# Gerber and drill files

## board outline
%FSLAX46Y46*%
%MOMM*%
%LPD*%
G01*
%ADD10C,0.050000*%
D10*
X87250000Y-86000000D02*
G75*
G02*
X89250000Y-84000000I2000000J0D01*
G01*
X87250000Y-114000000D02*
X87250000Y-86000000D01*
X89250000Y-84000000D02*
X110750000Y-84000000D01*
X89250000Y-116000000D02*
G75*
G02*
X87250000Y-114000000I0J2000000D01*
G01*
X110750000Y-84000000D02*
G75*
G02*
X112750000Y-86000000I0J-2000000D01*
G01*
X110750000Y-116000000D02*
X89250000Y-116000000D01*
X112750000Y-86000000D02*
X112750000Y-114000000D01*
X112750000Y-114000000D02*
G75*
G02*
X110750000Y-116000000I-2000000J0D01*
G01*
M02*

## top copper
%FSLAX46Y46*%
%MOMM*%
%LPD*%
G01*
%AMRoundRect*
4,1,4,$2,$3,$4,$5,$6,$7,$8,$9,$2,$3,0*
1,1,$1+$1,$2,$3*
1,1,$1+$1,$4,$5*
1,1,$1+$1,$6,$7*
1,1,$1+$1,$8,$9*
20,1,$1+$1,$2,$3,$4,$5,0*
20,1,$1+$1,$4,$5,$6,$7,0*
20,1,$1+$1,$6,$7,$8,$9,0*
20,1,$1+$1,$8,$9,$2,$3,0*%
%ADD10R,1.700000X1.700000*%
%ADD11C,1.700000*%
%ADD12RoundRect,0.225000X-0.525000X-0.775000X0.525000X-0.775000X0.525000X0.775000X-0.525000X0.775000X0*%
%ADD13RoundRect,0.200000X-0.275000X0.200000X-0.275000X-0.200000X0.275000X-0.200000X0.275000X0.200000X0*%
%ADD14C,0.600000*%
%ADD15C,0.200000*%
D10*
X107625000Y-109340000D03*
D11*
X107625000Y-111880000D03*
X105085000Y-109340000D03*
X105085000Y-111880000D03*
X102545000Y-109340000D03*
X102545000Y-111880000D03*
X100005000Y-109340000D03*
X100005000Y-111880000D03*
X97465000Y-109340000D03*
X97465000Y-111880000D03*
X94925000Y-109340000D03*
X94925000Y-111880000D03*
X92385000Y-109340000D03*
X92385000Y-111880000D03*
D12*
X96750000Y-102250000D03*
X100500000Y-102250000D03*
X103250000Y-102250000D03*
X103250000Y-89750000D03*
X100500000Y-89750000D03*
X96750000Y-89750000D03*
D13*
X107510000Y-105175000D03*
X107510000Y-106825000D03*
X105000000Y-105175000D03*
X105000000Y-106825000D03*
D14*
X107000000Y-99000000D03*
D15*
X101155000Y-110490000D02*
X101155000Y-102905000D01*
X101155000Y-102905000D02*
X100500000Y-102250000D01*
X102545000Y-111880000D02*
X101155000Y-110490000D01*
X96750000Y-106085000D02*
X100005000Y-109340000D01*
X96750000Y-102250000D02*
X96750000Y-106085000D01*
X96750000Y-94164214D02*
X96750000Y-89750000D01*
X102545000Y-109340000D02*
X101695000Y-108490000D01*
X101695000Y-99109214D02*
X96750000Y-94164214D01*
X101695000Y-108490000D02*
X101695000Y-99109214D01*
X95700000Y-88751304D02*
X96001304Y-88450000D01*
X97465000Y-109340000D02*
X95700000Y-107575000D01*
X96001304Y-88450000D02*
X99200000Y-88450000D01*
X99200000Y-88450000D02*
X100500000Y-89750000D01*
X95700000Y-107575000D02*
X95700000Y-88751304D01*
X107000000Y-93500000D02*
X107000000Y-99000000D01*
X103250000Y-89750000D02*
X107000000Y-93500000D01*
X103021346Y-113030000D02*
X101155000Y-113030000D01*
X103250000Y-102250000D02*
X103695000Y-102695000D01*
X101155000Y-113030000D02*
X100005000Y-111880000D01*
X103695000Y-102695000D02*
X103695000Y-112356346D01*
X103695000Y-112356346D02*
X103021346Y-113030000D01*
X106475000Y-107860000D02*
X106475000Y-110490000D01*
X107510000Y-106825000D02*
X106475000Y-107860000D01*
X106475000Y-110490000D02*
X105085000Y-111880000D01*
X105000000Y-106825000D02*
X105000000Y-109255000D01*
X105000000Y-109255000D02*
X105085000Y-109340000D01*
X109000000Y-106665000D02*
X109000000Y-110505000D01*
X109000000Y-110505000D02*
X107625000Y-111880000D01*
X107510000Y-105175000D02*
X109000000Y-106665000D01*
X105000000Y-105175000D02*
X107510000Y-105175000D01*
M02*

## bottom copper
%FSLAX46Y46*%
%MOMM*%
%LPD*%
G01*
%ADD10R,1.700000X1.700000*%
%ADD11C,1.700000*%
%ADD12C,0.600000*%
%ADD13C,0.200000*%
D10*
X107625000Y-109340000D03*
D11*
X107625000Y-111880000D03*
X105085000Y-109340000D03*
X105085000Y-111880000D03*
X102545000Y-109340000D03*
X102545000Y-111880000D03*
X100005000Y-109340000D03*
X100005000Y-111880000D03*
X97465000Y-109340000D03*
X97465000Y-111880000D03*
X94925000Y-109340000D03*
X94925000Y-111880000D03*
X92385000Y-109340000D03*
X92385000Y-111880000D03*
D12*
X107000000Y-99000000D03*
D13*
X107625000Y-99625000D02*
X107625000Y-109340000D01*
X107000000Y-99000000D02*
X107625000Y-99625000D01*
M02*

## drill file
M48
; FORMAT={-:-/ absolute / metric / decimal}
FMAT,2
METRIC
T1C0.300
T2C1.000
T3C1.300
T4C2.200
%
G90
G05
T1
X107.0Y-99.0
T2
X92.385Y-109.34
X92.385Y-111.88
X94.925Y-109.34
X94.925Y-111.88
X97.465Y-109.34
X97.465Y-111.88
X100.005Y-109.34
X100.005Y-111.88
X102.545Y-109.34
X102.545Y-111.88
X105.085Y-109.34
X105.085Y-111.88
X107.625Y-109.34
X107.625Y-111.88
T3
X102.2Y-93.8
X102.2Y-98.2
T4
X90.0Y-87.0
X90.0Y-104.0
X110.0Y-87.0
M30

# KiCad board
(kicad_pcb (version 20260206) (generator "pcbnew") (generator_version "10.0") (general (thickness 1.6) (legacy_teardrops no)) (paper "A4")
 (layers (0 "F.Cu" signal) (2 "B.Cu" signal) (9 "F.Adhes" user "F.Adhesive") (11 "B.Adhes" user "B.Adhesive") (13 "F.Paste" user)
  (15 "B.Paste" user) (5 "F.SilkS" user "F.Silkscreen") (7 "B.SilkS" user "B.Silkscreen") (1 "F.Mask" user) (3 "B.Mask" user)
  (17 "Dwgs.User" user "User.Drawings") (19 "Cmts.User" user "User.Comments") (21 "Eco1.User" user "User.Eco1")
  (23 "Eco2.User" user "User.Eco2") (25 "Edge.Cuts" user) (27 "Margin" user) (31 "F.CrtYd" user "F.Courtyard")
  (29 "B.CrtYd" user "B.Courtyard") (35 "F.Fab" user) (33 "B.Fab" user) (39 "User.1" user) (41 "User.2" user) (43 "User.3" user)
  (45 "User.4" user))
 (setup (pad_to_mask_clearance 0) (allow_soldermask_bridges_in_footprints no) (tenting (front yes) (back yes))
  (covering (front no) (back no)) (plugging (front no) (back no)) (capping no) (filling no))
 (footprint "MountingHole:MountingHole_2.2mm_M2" (layer "F.Cu") (at 90 87)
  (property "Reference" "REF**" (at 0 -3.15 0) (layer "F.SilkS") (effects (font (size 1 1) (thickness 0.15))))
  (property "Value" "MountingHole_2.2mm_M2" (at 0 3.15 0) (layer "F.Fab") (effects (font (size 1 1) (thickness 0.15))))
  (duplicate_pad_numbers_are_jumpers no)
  (pad "" np_thru_hole circle (at 0 0) (size 2.2 2.2) (drill 2.2) (layers "*.Cu" "*.Mask")))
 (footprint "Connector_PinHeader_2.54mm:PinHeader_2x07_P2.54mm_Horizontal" (layer "F.Cu") (at 107.625 109.34 -90)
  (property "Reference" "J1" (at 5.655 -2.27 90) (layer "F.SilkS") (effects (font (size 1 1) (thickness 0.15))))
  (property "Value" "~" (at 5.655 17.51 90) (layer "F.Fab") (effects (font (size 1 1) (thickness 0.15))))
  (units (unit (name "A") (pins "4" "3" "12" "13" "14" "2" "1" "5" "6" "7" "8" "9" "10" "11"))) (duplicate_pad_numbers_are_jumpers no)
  (pad "1" thru_hole rect (at 0 0 270) (size 1.7 1.7) (drill 1) (layers "*.Cu" "*.Mask") (remove_unused_layers no) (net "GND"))
  (pad "2" thru_hole circle (at 2.54 0 270) (size 1.7 1.7) (drill 1) (layers "*.Cu" "*.Mask") (remove_unused_layers no) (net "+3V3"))
  (pad "3" thru_hole circle (at 0 2.54 270) (size 1.7 1.7) (drill 1) (layers "*.Cu" "*.Mask") (remove_unused_layers no) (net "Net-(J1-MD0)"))
  (pad "4" thru_hole circle (at 2.54 2.54 270) (size 1.7 1.7) (drill 1) (layers "*.Cu" "*.Mask") (remove_unused_layers no)
   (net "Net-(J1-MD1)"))
  (pad "5" thru_hole circle (at 0 5.08 270) (size 1.7 1.7) (drill 1) (layers "*.Cu" "*.Mask") (remove_unused_layers no)
   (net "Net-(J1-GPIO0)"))
  (pad "6" thru_hole circle (at 2.54 5.08 270) (size 1.7 1.7) (drill 1) (layers "*.Cu" "*.Mask") (remove_unused_layers no)
   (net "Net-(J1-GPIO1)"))
  (pad "7" thru_hole circle (at 0 7.62 270) (size 1.7 1.7) (drill 1) (layers "*.Cu" "*.Mask") (remove_unused_layers no)
   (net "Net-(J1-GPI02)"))
  (pad "8" thru_hole circle (at 2.54 7.62 270) (size 1.7 1.7) (drill 1) (layers "*.Cu" "*.Mask") (remove_unused_layers no)
   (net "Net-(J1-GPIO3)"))
  (pad "9" thru_hole circle (at 0 10.16 270) (size 1.7 1.7) (drill 1) (layers "*.Cu" "*.Mask") (remove_unused_layers no)
   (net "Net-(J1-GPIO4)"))
  (pad "10" thru_hole circle (at 2.54 10.16 270) (size 1.7 1.7) (drill 1) (layers "*.Cu" "*.Mask") (remove_unused_layers no)
   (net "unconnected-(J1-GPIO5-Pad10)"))
  (pad "11" thru_hole circle (at 0 12.7 270) (size 1.7 1.7) (drill 1) (layers "*.Cu" "*.Mask") (remove_unused_layers no)
   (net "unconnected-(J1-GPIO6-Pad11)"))
  (pad "12" thru_hole circle (at 2.54 12.7 270) (size 1.7 1.7) (drill 1) (layers "*.Cu" "*.Mask") (remove_unused_layers no)
   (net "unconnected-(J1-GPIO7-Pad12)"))
  (pad "13" thru_hole circle (at 0 15.24 270) (size 1.7 1.7) (drill 1) (layers "*.Cu" "*.Mask") (remove_unused_layers no)
   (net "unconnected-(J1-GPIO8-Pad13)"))
  (pad "14" thru_hole circle (at 2.54 15.24 270) (size 1.7 1.7) (drill 1) (layers "*.Cu" "*.Mask") (remove_unused_layers no)
   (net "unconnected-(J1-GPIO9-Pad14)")))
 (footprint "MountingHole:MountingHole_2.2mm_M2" (layer "F.Cu") (at 110 87)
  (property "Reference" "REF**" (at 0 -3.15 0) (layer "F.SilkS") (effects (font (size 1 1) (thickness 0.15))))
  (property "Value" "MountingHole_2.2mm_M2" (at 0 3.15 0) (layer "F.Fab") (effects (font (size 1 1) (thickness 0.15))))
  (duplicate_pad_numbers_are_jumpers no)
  (pad "" np_thru_hole circle (at 0 0) (size 2.2 2.2) (drill 2.2) (layers "*.Cu" "*.Mask")))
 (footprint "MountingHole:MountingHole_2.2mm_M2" (layer "F.Cu") (at 90 104)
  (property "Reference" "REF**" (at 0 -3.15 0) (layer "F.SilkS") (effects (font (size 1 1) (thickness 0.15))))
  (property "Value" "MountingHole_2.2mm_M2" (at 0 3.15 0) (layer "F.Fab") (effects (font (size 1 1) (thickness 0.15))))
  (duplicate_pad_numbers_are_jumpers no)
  (pad "" np_thru_hole circle (at 0 0) (size 2.2 2.2) (drill 2.2) (layers "*.Cu" "*.Mask")))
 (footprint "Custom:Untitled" (layer "F.Cu") (at 100 96)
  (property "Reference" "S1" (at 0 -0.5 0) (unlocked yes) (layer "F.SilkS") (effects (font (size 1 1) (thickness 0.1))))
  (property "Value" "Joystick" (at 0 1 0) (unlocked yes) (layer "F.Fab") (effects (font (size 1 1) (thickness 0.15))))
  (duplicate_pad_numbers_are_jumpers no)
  (pad "" np_thru_hole circle (at 2.2 -2.2) (size 1.3 1.3) (drill 1.3) (layers "*.Mask"))
  (pad "" np_thru_hole circle (at 2.2 2.2) (size 1.3 1.3) (drill 1.3) (layers "*.Mask"))
  (pad "1" smd roundrect (at -3.25 6.25) (size 1.5 2) (layers "F.Cu" "F.Mask" "F.Paste") (roundrect_rratio 0.15) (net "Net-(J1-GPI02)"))
  (pad "2" smd roundrect (at 0.5 6.25) (size 1.5 2) (layers "F.Cu" "F.Mask" "F.Paste") (roundrect_rratio 0.15) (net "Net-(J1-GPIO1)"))
  (pad "3" smd roundrect (at 3.25 6.25) (size 1.5 2) (layers "F.Cu" "F.Mask" "F.Paste") (roundrect_rratio 0.15) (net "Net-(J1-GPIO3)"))
  (pad "4" smd roundrect (at 3.25 -6.25) (size 1.5 2) (layers "F.Cu" "F.Mask" "F.Paste") (roundrect_rratio 0.15) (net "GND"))
  (pad "5" smd roundrect (at 0.5 -6.25) (size 1.5 2) (layers "F.Cu" "F.Mask" "F.Paste") (roundrect_rratio 0.15) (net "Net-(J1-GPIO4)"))
  (pad "6" smd roundrect (at -3.25 -6.25) (size 1.5 2) (layers "F.Cu" "F.Mask" "F.Paste") (roundrect_rratio 0.15) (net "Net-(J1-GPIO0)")))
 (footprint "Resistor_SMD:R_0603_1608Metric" (layer "F.Cu") (at 107.51 106 -90)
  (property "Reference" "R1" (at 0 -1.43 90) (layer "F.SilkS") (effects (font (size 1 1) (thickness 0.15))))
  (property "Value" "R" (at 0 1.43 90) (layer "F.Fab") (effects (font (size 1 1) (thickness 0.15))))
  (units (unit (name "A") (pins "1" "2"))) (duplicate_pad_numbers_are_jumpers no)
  (pad "1" smd roundrect (at -0.825 0 270) (size 0.8 0.95) (layers "F.Cu" "F.Mask" "F.Paste") (roundrect_rratio 0.25) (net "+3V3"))
  (pad "2" smd roundrect (at 0.825 0 270) (size 0.8 0.95) (layers "F.Cu" "F.Mask" "F.Paste") (roundrect_rratio 0.25) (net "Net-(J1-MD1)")))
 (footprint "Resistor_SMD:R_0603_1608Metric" (layer "F.Cu") (at 105 106 -90)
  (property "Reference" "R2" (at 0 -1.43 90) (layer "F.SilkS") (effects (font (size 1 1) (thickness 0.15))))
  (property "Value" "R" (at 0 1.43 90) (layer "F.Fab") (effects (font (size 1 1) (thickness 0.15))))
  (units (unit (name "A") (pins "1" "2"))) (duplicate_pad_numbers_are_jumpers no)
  (pad "1" smd roundrect (at -0.825 0 270) (size 0.8 0.95) (layers "F.Cu" "F.Mask" "F.Paste") (roundrect_rratio 0.25) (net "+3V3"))
  (pad "2" smd roundrect (at 0.825 0 270) (size 0.8 0.95) (layers "F.Cu" "F.Mask" "F.Paste") (roundrect_rratio 0.25) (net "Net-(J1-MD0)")))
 (gr_arc (start 87.25 86) (mid 87.835786 84.585786) (end 89.25 84) (stroke (width 0.05) (type default)) (layer "Edge.Cuts"))
 (gr_line (start 87.25 114) (end 87.25 86) (stroke (width 0.05) (type default)) (layer "Edge.Cuts"))
 (gr_line (start 89.25 84) (end 110.75 84) (stroke (width 0.05) (type default)) (layer "Edge.Cuts"))
 (gr_arc (start 89.25 116) (mid 87.835786 115.414214) (end 87.25 114) (stroke (width 0.05) (type default)) (layer "Edge.Cuts"))
 (gr_arc (start 110.75 84) (mid 112.164214 84.585786) (end 112.75 86) (stroke (width 0.05) (type default)) (layer "Edge.Cuts"))
 (gr_line (start 110.75 116) (end 89.25 116) (stroke (width 0.05) (type default)) (layer "Edge.Cuts"))
 (gr_line (start 112.75 86) (end 112.75 114) (stroke (width 0.05) (type default)) (layer "Edge.Cuts"))
 (gr_arc (start 112.75 114) (mid 112.164214 115.414214) (end 110.75 116) (stroke (width 0.05) (type default)) (layer "Edge.Cuts"))
 (segment (start 101.155 110.49) (end 101.155 102.905) (width 0.2) (layer "F.Cu") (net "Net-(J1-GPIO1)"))
 (segment (start 101.155 102.905) (end 100.5 102.25) (width 0.2) (layer "F.Cu") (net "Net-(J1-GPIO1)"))
 (segment (start 102.545 111.88) (end 101.155 110.49) (width 0.2) (layer "F.Cu") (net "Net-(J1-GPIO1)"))
 (segment (start 96.75 106.085) (end 100.005 109.34) (width 0.2) (layer "F.Cu") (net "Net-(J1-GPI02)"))
 (segment (start 96.75 102.25) (end 96.75 106.085) (width 0.2) (layer "F.Cu") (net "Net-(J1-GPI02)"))
 (segment (start 96.75 94.164214) (end 96.75 89.75) (width 0.2) (layer "F.Cu") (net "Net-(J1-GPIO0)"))
 (segment (start 102.545 109.34) (end 101.695 108.49) (width 0.2) (layer "F.Cu") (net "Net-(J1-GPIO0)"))
 (segment (start 101.695 99.109214) (end 96.75 94.164214) (width 0.2) (layer "F.Cu") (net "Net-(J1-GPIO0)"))
 (segment (start 101.695 108.49) (end 101.695 99.109214) (width 0.2) (layer "F.Cu") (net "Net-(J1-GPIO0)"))
 (segment (start 95.7 88.751304) (end 96.001304 88.45) (width 0.2) (layer "F.Cu") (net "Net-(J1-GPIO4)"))
 (segment (start 97.465 109.34) (end 95.7 107.575) (width 0.2) (layer "F.Cu") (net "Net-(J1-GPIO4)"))
 (segment (start 96.001304 88.45) (end 99.2 88.45) (width 0.2) (layer "F.Cu") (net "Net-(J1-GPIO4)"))
 (segment (start 99.2 88.45) (end 100.5 89.75) (width 0.2) (layer "F.Cu") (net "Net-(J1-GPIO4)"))
 (segment (start 95.7 107.575) (end 95.7 88.751304) (width 0.2) (layer "F.Cu") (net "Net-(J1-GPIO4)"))
 (segment (start 107 93.5) (end 107 99) (width 0.2) (layer "F.Cu") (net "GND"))
 (segment (start 103.25 89.75) (end 107 93.5) (width 0.2) (layer "F.Cu") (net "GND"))
 (via (at 107 99) (size 0.6) (drill 0.3) (layers "F.Cu" "B.Cu") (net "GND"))
 (segment (start 107.625 99.625) (end 107.625 109.34) (width 0.2) (layer "B.Cu") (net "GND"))
 (segment (start 107 99) (end 107.625 99.625) (width 0.2) (layer "B.Cu") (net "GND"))
 (segment (start 103.021346 113.03) (end 101.155 113.03) (width 0.2) (layer "F.Cu") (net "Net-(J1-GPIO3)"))
 (segment (start 103.25 102.25) (end 103.695 102.695) (width 0.2) (layer "F.Cu") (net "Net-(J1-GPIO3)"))
 (segment (start 101.155 113.03) (end 100.005 111.88) (width 0.2) (layer "F.Cu") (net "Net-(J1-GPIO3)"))
 (segment (start 103.695 102.695) (end 103.695 112.356346) (width 0.2) (layer "F.Cu") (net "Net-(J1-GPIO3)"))
 (segment (start 103.695 112.356346) (end 103.021346 113.03) (width 0.2) (layer "F.Cu") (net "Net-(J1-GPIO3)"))
 (segment (start 106.475 107.86) (end 106.475 110.49) (width 0.2) (layer "F.Cu") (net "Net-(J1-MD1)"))
 (segment (start 107.51 106.825) (end 106.475 107.86) (width 0.2) (layer "F.Cu") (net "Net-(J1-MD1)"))
 (segment (start 106.475 110.49) (end 105.085 111.88) (width 0.2) (layer "F.Cu") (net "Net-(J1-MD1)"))
 (segment (start 105 106.825) (end 105 109.255) (width 0.2) (layer "F.Cu") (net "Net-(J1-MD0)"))
 (segment (start 105 109.255) (end 105.085 109.34) (width 0.2) (layer "F.Cu") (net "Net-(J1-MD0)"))
 (segment (start 109 106.665) (end 109 110.505) (width 0.2) (layer "F.Cu") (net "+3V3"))
 (segment (start 109 110.505) (end 107.625 111.88) (width 0.2) (layer "F.Cu") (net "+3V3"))
 (segment (start 107.51 105.175) (end 109 106.665) (width 0.2) (layer "F.Cu") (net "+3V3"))
 (segment (start 105 105.175) (end 107.51 105.175) (width 0.2) (layer "F.Cu") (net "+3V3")))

